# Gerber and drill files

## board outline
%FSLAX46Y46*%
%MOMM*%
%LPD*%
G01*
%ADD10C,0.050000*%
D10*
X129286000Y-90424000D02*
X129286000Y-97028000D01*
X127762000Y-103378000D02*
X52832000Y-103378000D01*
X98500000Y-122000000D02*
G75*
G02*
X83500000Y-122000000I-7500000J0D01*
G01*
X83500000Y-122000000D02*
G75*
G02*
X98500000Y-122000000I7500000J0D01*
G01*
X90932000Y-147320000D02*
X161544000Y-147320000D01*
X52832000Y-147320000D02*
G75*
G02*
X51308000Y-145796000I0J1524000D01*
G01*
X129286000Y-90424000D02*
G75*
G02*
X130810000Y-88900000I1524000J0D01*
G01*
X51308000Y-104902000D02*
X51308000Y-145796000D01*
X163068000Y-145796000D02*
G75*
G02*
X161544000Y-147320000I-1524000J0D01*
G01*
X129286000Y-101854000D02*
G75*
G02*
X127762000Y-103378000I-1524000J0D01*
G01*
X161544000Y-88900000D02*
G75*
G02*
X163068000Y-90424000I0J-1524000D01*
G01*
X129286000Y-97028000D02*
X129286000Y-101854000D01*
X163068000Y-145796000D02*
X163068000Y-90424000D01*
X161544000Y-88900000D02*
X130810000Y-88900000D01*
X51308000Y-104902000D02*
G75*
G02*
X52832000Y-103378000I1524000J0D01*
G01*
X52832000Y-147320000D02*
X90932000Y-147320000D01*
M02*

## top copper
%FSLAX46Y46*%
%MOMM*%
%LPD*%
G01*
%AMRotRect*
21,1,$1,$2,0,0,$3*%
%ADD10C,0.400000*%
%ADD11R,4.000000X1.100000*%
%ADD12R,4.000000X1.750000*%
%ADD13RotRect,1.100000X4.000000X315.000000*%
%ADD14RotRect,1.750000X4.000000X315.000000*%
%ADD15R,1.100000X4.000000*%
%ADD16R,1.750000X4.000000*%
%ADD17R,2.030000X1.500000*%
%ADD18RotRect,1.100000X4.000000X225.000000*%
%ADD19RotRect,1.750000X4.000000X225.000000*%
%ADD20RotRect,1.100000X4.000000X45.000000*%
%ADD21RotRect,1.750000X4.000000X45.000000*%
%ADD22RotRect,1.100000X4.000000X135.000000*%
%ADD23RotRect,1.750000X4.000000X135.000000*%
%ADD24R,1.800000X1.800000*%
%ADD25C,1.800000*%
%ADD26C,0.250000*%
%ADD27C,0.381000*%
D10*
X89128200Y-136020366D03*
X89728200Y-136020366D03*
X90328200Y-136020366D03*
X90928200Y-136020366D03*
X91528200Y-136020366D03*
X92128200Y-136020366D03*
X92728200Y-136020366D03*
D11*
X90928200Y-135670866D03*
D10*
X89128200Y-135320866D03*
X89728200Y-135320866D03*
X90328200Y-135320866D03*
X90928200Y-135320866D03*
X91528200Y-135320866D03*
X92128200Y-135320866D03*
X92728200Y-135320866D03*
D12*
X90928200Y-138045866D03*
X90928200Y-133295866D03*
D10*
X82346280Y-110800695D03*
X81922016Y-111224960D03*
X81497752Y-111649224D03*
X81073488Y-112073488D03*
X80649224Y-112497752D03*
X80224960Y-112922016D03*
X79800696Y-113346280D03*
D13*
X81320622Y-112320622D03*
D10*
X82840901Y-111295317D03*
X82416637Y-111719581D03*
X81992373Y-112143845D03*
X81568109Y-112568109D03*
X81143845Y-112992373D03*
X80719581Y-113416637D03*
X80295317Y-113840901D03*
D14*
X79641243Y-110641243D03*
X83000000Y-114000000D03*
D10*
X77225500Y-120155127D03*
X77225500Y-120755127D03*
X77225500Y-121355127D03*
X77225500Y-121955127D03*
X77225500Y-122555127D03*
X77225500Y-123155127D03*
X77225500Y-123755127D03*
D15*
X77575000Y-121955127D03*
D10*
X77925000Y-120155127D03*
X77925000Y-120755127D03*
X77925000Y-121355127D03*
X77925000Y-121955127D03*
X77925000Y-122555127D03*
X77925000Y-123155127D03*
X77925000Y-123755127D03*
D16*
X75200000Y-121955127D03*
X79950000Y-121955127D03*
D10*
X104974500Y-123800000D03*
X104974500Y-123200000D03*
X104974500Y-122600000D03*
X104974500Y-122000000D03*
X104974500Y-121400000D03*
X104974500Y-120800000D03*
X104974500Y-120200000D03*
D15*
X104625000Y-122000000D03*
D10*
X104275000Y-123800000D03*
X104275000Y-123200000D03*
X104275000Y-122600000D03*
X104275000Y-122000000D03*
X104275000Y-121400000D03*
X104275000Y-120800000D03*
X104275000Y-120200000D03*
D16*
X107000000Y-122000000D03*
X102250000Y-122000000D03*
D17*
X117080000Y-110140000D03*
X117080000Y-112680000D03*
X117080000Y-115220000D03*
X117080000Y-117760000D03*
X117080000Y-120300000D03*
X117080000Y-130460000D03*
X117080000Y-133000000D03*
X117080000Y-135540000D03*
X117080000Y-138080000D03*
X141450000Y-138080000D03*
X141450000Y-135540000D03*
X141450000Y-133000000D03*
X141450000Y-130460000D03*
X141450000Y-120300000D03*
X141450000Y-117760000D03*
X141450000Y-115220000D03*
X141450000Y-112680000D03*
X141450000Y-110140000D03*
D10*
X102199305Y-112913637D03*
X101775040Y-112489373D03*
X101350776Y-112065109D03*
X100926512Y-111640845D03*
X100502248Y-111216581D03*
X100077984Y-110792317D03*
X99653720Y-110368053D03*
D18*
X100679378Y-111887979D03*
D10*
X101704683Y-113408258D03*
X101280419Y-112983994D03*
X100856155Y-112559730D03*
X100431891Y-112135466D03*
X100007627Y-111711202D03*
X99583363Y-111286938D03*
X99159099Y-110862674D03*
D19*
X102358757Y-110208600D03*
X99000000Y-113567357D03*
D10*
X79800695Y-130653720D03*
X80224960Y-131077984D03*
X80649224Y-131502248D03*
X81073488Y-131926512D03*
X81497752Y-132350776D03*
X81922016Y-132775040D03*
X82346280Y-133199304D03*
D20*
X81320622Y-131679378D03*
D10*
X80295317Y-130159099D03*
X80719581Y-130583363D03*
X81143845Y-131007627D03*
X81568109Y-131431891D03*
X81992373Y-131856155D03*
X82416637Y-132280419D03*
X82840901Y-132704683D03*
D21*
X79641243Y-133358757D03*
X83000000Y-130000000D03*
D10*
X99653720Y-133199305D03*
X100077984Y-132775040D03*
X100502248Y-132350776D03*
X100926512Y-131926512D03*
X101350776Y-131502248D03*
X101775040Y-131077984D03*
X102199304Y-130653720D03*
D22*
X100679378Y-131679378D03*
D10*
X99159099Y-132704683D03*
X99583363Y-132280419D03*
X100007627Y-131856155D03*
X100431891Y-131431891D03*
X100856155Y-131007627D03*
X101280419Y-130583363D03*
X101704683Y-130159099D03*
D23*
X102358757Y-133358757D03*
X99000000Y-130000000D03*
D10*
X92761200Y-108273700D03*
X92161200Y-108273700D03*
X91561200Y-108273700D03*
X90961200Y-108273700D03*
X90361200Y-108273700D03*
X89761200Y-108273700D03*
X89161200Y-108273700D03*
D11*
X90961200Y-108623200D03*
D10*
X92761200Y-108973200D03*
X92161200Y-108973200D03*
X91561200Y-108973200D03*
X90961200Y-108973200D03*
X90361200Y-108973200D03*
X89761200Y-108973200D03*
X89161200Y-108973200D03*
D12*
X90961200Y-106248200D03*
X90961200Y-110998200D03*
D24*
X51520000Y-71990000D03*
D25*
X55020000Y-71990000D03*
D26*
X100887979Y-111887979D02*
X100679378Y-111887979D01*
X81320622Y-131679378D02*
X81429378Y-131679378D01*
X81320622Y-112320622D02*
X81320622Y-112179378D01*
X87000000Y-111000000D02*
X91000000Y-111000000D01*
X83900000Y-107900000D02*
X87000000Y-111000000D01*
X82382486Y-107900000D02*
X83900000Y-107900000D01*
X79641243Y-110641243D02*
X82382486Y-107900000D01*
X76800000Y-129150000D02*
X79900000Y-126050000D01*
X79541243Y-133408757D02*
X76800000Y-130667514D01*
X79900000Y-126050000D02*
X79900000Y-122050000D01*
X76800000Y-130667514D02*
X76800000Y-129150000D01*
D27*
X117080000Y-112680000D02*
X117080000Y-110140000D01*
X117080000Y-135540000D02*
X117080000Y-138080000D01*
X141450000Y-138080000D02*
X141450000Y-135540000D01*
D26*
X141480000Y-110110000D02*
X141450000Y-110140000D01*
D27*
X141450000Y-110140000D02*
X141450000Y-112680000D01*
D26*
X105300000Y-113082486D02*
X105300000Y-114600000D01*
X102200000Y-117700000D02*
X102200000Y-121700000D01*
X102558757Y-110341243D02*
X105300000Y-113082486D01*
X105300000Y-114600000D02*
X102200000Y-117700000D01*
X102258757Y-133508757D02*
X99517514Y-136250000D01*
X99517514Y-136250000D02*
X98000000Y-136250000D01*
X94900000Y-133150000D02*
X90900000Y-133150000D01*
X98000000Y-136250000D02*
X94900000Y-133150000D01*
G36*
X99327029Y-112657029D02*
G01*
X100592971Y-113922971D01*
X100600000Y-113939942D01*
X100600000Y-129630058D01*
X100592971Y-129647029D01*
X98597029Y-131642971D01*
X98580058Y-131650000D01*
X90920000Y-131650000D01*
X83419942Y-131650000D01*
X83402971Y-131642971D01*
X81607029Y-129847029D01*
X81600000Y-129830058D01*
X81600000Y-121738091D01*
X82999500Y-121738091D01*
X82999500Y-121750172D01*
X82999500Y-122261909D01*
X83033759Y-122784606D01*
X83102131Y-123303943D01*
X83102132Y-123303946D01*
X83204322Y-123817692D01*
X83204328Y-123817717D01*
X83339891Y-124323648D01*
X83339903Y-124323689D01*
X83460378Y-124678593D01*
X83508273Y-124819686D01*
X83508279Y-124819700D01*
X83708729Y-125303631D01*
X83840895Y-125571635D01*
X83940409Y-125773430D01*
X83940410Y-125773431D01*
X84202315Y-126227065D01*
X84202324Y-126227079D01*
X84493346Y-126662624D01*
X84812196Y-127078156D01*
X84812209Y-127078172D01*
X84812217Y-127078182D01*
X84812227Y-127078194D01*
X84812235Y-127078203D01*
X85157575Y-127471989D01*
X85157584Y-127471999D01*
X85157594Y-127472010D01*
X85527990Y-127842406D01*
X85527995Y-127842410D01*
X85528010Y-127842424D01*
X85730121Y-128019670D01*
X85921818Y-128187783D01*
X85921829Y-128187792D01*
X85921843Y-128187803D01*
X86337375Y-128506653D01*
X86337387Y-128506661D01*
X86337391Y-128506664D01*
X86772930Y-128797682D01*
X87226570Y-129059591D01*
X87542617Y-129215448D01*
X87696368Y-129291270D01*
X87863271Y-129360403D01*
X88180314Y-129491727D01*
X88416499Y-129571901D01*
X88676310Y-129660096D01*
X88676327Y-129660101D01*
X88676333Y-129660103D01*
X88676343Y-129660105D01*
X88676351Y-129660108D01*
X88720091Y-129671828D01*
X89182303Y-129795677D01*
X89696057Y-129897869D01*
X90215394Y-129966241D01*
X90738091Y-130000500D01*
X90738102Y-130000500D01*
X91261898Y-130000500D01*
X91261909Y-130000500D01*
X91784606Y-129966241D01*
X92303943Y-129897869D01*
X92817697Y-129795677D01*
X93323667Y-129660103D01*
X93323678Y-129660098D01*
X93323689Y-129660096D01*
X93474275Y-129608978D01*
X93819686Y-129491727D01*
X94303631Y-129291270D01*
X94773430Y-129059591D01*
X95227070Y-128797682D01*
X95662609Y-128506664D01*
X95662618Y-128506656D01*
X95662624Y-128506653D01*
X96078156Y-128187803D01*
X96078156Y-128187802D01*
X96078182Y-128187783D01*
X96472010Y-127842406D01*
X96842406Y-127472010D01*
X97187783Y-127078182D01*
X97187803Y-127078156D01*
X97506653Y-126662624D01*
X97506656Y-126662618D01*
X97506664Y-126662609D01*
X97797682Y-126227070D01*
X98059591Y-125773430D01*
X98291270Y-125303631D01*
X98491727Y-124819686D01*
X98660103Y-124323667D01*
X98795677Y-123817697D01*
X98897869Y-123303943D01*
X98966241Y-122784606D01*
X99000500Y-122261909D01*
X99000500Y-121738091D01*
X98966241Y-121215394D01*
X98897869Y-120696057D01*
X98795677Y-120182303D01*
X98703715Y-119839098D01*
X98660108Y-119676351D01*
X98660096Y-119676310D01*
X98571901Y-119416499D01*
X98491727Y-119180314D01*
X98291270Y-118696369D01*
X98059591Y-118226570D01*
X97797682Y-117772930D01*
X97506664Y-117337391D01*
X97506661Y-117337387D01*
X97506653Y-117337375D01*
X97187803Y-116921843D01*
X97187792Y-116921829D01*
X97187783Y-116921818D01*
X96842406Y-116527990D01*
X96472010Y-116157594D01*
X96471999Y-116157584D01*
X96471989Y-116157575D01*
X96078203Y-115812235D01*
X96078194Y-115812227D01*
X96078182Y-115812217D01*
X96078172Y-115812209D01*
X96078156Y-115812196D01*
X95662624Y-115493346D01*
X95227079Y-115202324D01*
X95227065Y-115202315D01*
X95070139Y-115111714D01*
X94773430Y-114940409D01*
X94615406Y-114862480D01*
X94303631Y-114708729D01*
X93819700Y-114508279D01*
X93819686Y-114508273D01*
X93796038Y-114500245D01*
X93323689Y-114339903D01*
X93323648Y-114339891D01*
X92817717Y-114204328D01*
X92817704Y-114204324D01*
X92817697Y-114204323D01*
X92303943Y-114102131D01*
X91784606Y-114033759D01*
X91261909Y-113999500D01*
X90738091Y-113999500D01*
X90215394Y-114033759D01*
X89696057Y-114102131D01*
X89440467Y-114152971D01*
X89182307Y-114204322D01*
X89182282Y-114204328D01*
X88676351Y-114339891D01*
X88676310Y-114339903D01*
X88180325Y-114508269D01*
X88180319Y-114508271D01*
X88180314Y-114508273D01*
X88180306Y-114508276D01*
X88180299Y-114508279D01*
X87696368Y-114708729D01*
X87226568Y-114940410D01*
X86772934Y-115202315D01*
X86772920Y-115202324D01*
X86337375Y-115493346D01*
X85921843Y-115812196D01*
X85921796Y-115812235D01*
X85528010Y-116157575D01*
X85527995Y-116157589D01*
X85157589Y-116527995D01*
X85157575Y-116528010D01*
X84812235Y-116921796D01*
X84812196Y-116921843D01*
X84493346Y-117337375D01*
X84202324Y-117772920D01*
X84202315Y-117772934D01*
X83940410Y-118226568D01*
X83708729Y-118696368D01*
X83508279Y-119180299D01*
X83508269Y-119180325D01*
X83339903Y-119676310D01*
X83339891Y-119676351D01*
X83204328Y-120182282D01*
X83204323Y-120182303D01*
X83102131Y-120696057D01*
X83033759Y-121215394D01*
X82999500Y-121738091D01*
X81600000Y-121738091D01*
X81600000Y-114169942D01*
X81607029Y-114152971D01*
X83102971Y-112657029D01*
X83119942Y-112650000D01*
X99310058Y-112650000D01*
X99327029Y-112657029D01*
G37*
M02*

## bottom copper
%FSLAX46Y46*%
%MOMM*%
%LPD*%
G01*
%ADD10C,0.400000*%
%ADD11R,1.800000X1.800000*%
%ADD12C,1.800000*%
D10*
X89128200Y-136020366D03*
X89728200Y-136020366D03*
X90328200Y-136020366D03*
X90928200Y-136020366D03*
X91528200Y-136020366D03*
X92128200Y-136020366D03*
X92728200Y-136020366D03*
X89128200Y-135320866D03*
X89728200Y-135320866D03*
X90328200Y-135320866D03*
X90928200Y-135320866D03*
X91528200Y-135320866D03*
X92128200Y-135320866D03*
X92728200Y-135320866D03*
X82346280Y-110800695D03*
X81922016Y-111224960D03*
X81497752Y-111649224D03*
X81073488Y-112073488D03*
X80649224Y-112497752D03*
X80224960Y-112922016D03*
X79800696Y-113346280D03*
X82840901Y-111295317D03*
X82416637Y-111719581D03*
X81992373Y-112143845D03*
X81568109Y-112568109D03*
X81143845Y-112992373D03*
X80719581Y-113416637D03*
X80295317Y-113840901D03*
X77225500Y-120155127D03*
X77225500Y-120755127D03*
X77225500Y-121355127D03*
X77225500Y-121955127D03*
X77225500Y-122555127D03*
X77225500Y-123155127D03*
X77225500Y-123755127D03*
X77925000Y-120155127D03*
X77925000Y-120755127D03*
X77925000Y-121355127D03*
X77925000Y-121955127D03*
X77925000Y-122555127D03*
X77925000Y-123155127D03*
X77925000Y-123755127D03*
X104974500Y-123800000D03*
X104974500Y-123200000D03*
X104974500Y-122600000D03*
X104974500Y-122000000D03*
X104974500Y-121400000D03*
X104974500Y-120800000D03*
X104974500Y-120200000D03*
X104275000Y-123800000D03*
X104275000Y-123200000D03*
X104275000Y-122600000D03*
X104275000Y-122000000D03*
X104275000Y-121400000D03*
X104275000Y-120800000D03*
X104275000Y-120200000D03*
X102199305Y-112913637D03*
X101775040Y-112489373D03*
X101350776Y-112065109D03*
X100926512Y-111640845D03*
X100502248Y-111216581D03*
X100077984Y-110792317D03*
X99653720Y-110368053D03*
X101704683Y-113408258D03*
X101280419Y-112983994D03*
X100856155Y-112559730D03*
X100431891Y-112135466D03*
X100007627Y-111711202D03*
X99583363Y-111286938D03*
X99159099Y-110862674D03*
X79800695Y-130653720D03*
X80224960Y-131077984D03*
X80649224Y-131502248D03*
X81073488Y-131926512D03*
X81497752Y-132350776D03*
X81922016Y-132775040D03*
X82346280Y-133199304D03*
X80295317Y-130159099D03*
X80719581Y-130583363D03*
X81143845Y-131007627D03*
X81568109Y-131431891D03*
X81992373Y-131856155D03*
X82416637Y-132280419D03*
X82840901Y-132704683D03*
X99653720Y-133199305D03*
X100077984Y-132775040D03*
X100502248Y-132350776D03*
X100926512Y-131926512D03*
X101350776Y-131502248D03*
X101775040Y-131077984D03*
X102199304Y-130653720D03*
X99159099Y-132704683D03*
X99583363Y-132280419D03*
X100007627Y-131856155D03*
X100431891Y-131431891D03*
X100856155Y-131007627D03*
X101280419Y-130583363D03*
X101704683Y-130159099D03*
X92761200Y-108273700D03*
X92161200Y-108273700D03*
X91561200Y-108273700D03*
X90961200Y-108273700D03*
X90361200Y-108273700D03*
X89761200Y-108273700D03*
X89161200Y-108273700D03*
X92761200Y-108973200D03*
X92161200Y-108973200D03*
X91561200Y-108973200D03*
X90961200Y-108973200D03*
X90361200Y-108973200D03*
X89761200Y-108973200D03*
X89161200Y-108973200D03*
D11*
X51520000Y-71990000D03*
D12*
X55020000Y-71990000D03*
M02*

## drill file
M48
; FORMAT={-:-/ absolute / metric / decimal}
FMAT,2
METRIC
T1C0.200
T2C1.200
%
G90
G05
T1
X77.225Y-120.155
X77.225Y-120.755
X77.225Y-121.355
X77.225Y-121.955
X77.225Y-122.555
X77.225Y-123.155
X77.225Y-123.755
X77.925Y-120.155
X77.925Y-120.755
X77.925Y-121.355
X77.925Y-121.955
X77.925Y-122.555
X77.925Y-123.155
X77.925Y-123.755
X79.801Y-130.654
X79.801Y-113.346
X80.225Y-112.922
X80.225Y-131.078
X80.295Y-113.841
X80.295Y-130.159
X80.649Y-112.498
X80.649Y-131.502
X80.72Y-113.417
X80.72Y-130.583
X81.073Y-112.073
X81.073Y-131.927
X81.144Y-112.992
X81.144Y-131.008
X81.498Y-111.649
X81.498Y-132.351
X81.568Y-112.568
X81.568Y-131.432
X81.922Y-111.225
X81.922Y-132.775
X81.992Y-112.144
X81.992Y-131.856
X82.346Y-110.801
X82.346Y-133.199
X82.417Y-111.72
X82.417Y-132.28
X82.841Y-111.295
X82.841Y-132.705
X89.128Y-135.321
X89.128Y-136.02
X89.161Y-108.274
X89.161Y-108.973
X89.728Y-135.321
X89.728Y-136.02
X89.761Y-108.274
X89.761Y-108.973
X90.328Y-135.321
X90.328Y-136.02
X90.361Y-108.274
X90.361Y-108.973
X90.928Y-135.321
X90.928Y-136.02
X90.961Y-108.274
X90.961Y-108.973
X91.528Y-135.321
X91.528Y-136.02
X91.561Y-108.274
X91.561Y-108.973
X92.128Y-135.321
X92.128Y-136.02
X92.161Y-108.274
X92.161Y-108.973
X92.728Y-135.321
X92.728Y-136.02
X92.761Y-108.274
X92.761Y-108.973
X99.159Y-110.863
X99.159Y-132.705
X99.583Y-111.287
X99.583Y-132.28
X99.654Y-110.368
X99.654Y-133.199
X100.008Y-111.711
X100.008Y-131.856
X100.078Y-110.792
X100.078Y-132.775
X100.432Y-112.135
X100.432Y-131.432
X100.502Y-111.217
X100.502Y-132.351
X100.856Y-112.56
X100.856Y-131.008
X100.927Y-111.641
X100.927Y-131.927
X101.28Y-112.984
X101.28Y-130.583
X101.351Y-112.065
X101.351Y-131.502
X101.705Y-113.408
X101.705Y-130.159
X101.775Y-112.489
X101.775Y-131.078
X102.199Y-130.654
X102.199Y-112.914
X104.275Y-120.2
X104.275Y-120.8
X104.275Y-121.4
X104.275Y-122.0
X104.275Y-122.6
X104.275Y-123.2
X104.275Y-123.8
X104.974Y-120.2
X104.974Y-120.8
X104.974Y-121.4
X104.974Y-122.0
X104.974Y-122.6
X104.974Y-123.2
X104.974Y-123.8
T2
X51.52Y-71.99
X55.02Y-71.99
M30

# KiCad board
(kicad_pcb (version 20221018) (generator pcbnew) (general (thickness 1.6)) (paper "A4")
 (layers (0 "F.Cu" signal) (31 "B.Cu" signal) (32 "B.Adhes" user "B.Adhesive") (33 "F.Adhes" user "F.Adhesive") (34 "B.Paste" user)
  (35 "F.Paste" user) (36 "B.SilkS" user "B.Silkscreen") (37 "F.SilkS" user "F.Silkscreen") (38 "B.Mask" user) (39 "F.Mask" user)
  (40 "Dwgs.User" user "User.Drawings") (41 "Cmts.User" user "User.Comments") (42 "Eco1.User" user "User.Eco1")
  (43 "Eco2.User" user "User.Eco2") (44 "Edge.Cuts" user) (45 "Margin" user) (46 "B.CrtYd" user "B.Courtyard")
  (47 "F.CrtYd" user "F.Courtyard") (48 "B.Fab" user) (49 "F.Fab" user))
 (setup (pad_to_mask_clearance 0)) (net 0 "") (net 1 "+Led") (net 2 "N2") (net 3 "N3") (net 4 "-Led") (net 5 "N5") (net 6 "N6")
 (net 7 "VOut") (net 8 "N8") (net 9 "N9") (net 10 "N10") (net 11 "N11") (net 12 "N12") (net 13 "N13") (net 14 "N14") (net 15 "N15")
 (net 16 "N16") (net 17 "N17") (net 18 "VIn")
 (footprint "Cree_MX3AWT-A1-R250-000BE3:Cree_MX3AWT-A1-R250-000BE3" (layer "F.Cu") (at 85.9282 138.045866 90)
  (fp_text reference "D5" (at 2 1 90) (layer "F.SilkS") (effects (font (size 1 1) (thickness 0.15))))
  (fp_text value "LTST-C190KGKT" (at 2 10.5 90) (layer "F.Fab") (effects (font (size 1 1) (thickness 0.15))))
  (pad "65" thru_hole circle (at 2.0255 3.2 90) (size 0.4 0.4) (drill 0.2) (layers "*.Cu" "B.Mask"))
  (pad "65" thru_hole circle (at 2.0255 3.8 90) (size 0.4 0.4) (drill 0.2) (layers "*.Cu" "B.Mask"))
  (pad "65" thru_hole circle (at 2.0255 4.4 90) (size 0.4 0.4) (drill 0.2) (layers "*.Cu" "B.Mask"))
  (pad "65" thru_hole circle (at 2.0255 5 90) (size 0.4 0.4) (drill 0.2) (layers "*.Cu" "B.Mask"))
  (pad "65" thru_hole circle (at 2.0255 5.6 90) (size 0.4 0.4) (drill 0.2) (layers "*.Cu" "B.Mask"))
  (pad "65" thru_hole circle (at 2.0255 6.2 90) (size 0.4 0.4) (drill 0.2) (layers "*.Cu" "B.Mask"))
  (pad "65" thru_hole circle (at 2.0255 6.8 90) (size 0.4 0.4) (drill 0.2) (layers "*.Cu" "B.Mask"))
  (pad "65" smd rect (at 2.375 5 90) (size 1.1 4) (layers "F.Cu" "F.Paste" "F.Mask"))
  (pad "65" thru_hole circle (at 2.725 3.2 90) (size 0.4 0.4) (drill 0.2) (layers "*.Cu" "B.Mask"))
  (pad "65" thru_hole circle (at 2.725 3.8 90) (size 0.4 0.4) (drill 0.2) (layers "*.Cu" "B.Mask"))
  (pad "65" thru_hole circle (at 2.725 4.4 90) (size 0.4 0.4) (drill 0.2) (layers "*.Cu" "B.Mask"))
  (pad "65" thru_hole circle (at 2.725 5 90) (size 0.4 0.4) (drill 0.2) (layers "*.Cu" "B.Mask"))
  (pad "65" thru_hole circle (at 2.725 5.6 90) (size 0.4 0.4) (drill 0.2) (layers "*.Cu" "B.Mask"))
  (pad "65" thru_hole circle (at 2.725 6.2 90) (size 0.4 0.4) (drill 0.2) (layers "*.Cu" "B.Mask"))
  (pad "65" thru_hole circle (at 2.725 6.8 90) (size 0.4 0.4) (drill 0.2) (layers "*.Cu" "B.Mask"))
  (pad "A" smd rect (at 0 5 90) (size 1.75 4) (layers "F.Cu" "F.Paste" "F.Mask") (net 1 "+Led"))
  (pad "C" smd rect (at 4.75 5 90) (size 1.75 4) (layers "F.Cu" "F.Paste" "F.Mask") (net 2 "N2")))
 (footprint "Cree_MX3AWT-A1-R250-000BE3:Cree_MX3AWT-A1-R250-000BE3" (layer "F.Cu") (at 83.176777 107.105709 -45)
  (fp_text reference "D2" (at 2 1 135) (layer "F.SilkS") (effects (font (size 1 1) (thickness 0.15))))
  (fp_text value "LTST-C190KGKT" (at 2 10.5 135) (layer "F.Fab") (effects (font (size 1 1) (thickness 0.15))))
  (pad "65" thru_hole circle (at 2.0255 3.2 315) (size 0.4 0.4) (drill 0.2) (layers "*.Cu" "B.Mask"))
  (pad "65" thru_hole circle (at 2.0255 3.8 315) (size 0.4 0.4) (drill 0.2) (layers "*.Cu" "B.Mask"))
  (pad "65" thru_hole circle (at 2.0255 4.4 315) (size 0.4 0.4) (drill 0.2) (layers "*.Cu" "B.Mask"))
  (pad "65" thru_hole circle (at 2.0255 5 315) (size 0.4 0.4) (drill 0.2) (layers "*.Cu" "B.Mask"))
  (pad "65" thru_hole circle (at 2.0255 5.6 315) (size 0.4 0.4) (drill 0.2) (layers "*.Cu" "B.Mask"))
  (pad "65" thru_hole circle (at 2.0255 6.2 315) (size 0.4 0.4) (drill 0.2) (layers "*.Cu" "B.Mask"))
  (pad "65" thru_hole circle (at 2.0255 6.8 315) (size 0.4 0.4) (drill 0.2) (layers "*.Cu" "B.Mask"))
  (pad "65" smd rect (at 2.375001 5 315) (size 1.1 4) (layers "F.Cu" "F.Paste" "F.Mask"))
  (pad "65" thru_hole circle (at 2.725 3.2 315) (size 0.4 0.4) (drill 0.2) (layers "*.Cu" "B.Mask"))
  (pad "65" thru_hole circle (at 2.725 3.8 315) (size 0.4 0.4) (drill 0.2) (layers "*.Cu" "B.Mask"))
  (pad "65" thru_hole circle (at 2.725 4.4 315) (size 0.4 0.4) (drill 0.2) (layers "*.Cu" "B.Mask"))
  (pad "65" thru_hole circle (at 2.725 5 315) (size 0.4 0.4) (drill 0.2) (layers "*.Cu" "B.Mask"))
  (pad "65" thru_hole circle (at 2.725 5.6 315) (size 0.4 0.4) (drill 0.2) (layers "*.Cu" "B.Mask"))
  (pad "65" thru_hole circle (at 2.725 6.2 315) (size 0.4 0.4) (drill 0.2) (layers "*.Cu" "B.Mask"))
  (pad "65" thru_hole circle (at 2.725 6.8 315) (size 0.4 0.4) (drill 0.2) (layers "*.Cu" "B.Mask"))
  (pad "A" smd rect (at 0 5 315) (size 1.75 4) (layers "F.Cu" "F.Paste" "F.Mask") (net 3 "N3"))
  (pad "C" smd rect (at 4.75 5 315) (size 1.75 4) (layers "F.Cu" "F.Paste" "F.Mask") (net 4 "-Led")))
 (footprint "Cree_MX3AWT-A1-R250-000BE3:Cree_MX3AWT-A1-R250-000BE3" (layer "F.Cu") (at 75.2 116.955127)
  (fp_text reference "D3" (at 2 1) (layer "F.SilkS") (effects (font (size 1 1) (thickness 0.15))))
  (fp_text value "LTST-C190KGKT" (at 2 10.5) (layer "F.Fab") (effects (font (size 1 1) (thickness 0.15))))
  (pad "65" thru_hole circle (at 2.0255 3.2) (size 0.4 0.4) (drill 0.2) (layers "*.Cu" "B.Mask"))
  (pad "65" thru_hole circle (at 2.0255 3.8) (size 0.4 0.4) (drill 0.2) (layers "*.Cu" "B.Mask"))
  (pad "65" thru_hole circle (at 2.0255 4.4) (size 0.4 0.4) (drill 0.2) (layers "*.Cu" "B.Mask"))
  (pad "65" thru_hole circle (at 2.0255 5) (size 0.4 0.4) (drill 0.2) (layers "*.Cu" "B.Mask"))
  (pad "65" thru_hole circle (at 2.0255 5.6) (size 0.4 0.4) (drill 0.2) (layers "*.Cu" "B.Mask"))
  (pad "65" thru_hole circle (at 2.0255 6.2) (size 0.4 0.4) (drill 0.2) (layers "*.Cu" "B.Mask"))
  (pad "65" thru_hole circle (at 2.0255 6.8) (size 0.4 0.4) (drill 0.2) (layers "*.Cu" "B.Mask"))
  (pad "65" smd rect (at 2.375 5) (size 1.1 4) (layers "F.Cu" "F.Paste" "F.Mask"))
  (pad "65" thru_hole circle (at 2.725 3.2) (size 0.4 0.4) (drill 0.2) (layers "*.Cu" "B.Mask"))
  (pad "65" thru_hole circle (at 2.725 3.8) (size 0.4 0.4) (drill 0.2) (layers "*.Cu" "B.Mask"))
  (pad "65" thru_hole circle (at 2.725 4.4) (size 0.4 0.4) (drill 0.2) (layers "*.Cu" "B.Mask"))
  (pad "65" thru_hole circle (at 2.725 5) (size 0.4 0.4) (drill 0.2) (layers "*.Cu" "B.Mask"))
  (pad "65" thru_hole circle (at 2.725 5.6) (size 0.4 0.4) (drill 0.2) (layers "*.Cu" "B.Mask"))
  (pad "65" thru_hole circle (at 2.725 6.2) (size 0.4 0.4) (drill 0.2) (layers "*.Cu" "B.Mask"))
  (pad "65" thru_hole circle (at 2.725 6.8) (size 0.4 0.4) (drill 0.2) (layers "*.Cu" "B.Mask"))
  (pad "A" smd rect (at 0 5) (size 1.75 4) (layers "F.Cu" "F.Paste" "F.Mask") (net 1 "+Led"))
  (pad "C" smd rect (at 4.75 5) (size 1.75 4) (layers "F.Cu" "F.Paste" "F.Mask") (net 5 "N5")))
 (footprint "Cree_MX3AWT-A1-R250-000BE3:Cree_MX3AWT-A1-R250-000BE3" (layer "F.Cu") (at 107 127 180)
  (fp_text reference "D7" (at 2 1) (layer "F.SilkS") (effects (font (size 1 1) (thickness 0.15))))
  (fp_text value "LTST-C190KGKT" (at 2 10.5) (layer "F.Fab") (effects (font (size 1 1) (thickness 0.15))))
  (pad "65" thru_hole circle (at 2.0255 3.2 180) (size 0.4 0.4) (drill 0.2) (layers "*.Cu" "B.Mask"))
  (pad "65" thru_hole circle (at 2.0255 3.8 180) (size 0.4 0.4) (drill 0.2) (layers "*.Cu" "B.Mask"))
  (pad "65" thru_hole circle (at 2.0255 4.4 180) (size 0.4 0.4) (drill 0.2) (layers "*.Cu" "B.Mask"))
  (pad "65" thru_hole circle (at 2.0255 5 180) (size 0.4 0.4) (drill 0.2) (layers "*.Cu" "B.Mask"))
  (pad "65" thru_hole circle (at 2.0255 5.6 180) (size 0.4 0.4) (drill 0.2) (layers "*.Cu" "B.Mask"))
  (pad "65" thru_hole circle (at 2.0255 6.2 180) (size 0.4 0.4) (drill 0.2) (layers "*.Cu" "B.Mask"))
  (pad "65" thru_hole circle (at 2.0255 6.8 180) (size 0.4 0.4) (drill 0.2) (layers "*.Cu" "B.Mask"))
  (pad "65" smd rect (at 2.375 5 180) (size 1.1 4) (layers "F.Cu" "F.Paste" "F.Mask"))
  (pad "65" thru_hole circle (at 2.725 3.2 180) (size 0.4 0.4) (drill 0.2) (layers "*.Cu" "B.Mask"))
  (pad "65" thru_hole circle (at 2.725 3.8 180) (size 0.4 0.4) (drill 0.2) (layers "*.Cu" "B.Mask"))
  (pad "65" thru_hole circle (at 2.725 4.4 180) (size 0.4 0.4) (drill 0.2) (layers "*.Cu" "B.Mask"))
  (pad "65" thru_hole circle (at 2.725 5 180) (size 0.4 0.4) (drill 0.2) (layers "*.Cu" "B.Mask"))
  (pad "65" thru_hole circle (at 2.725 5.6 180) (size 0.4 0.4) (drill 0.2) (layers "*.Cu" "B.Mask"))
  (pad "65" thru_hole circle (at 2.725 6.2 180) (size 0.4 0.4) (drill 0.2) (layers "*.Cu" "B.Mask"))
  (pad "65" thru_hole circle (at 2.725 6.8 180) (size 0.4 0.4) (drill 0.2) (layers "*.Cu" "B.Mask"))
  (pad "A" smd rect (at 0 5 180) (size 1.75 4) (layers "F.Cu" "F.Paste" "F.Mask") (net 1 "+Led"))
  (pad "C" smd rect (at 4.75 5 180) (size 1.75 4) (layers "F.Cu" "F.Paste" "F.Mask") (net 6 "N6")))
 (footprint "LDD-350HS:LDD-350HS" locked (layer "F.Cu") (at 117.08 105.64)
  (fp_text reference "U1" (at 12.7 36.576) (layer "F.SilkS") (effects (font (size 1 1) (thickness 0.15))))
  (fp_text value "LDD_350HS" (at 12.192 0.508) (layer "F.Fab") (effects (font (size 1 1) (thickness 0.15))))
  (pad "1" smd rect locked (at 0 4.5) (size 2.03 1.5) (layers "F.Cu" "F.Paste" "F.Mask") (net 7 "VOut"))
  (pad "2" smd rect locked (at 0 7.04) (size 2.03 1.5) (layers "F.Cu" "F.Paste" "F.Mask") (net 7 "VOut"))
  (pad "3" smd rect locked (at 0 9.58) (size 2.03 1.5) (layers "F.Cu" "F.Paste" "F.Mask") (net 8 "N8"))
  (pad "4" smd rect locked (at 0 12.12) (size 2.03 1.5) (layers "F.Cu" "F.Paste" "F.Mask") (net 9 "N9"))
  (pad "5" smd rect locked (at 0 14.66) (size 2.03 1.5) (layers "F.Cu" "F.Paste" "F.Mask") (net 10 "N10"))
  (pad "9" smd rect locked (at 0 24.82) (size 2.03 1.5) (layers "F.Cu" "F.Paste" "F.Mask") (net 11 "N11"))
  (pad "10" smd rect locked (at 0 27.36) (size 2.03 1.5) (layers "F.Cu" "F.Paste" "F.Mask") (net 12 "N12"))
  (pad "11" smd rect locked (at 0 29.9) (size 2.03 1.5) (layers "F.Cu" "F.Paste" "F.Mask") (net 4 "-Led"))
  (pad "12" smd rect locked (at 0 32.44) (size 2.03 1.5) (layers "F.Cu" "F.Paste" "F.Mask") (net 4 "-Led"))
  (pad "13" smd rect locked (at 24.37 32.44) (size 2.03 1.5) (layers "F.Cu" "F.Paste" "F.Mask") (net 1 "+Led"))
  (pad "14" smd rect locked (at 24.37 29.9) (size 2.03 1.5) (layers "F.Cu" "F.Paste" "F.Mask") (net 1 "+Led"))
  (pad "15" smd rect locked (at 24.37 27.36) (size 2.03 1.5) (layers "F.Cu" "F.Paste" "F.Mask") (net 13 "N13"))
  (pad "16" smd rect locked (at 24.37 24.82) (size 2.03 1.5) (layers "F.Cu" "F.Paste" "F.Mask") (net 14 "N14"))
  (pad "20" smd rect locked (at 24.37 14.66) (size 2.03 1.5) (layers "F.Cu" "F.Paste" "F.Mask") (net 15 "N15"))
  (pad "21" smd rect locked (at 24.37 12.12) (size 2.03 1.5) (layers "F.Cu" "F.Paste" "F.Mask") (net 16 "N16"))
  (pad "22" smd rect locked (at 24.37 9.58) (size 2.03 1.5) (layers "F.Cu" "F.Paste" "F.Mask") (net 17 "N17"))
  (pad "23" smd rect locked (at 24.37 7.04) (size 2.03 1.5) (layers "F.Cu" "F.Paste" "F.Mask") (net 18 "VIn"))
  (pad "24" smd rect locked (at 24.37 4.5) (size 2.03 1.5) (layers "F.Cu" "F.Paste" "F.Mask") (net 18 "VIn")))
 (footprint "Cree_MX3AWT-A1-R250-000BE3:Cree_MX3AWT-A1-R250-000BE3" (layer "F.Cu") (at 105.894291 113.744134 -135)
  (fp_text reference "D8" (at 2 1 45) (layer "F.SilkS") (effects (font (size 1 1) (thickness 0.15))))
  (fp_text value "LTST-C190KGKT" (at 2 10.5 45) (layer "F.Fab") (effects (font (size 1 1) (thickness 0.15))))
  (pad "65" thru_hole circle (at 2.0255 3.2 225) (size 0.4 0.4) (drill 0.2) (layers "*.Cu" "B.Mask"))
  (pad "65" thru_hole circle (at 2.0255 3.8 225) (size 0.4 0.4) (drill 0.2) (layers "*.Cu" "B.Mask"))
  (pad "65" thru_hole circle (at 2.0255 4.4 225) (size 0.4 0.4) (drill 0.2) (layers "*.Cu" "B.Mask"))
  (pad "65" thru_hole circle (at 2.0255 5 225) (size 0.4 0.4) (drill 0.2) (layers "*.Cu" "B.Mask"))
  (pad "65" thru_hole circle (at 2.0255 5.6 225) (size 0.4 0.4) (drill 0.2) (layers "*.Cu" "B.Mask"))
  (pad "65" thru_hole circle (at 2.0255 6.2 225) (size 0.4 0.4) (drill 0.2) (layers "*.Cu" "B.Mask"))
  (pad "65" thru_hole circle (at 2.0255 6.8 225) (size 0.4 0.4) (drill 0.2) (layers "*.Cu" "B.Mask"))
  (pad "65" smd rect (at 2.375001 5 225) (size 1.1 4) (layers "F.Cu" "F.Paste" "F.Mask"))
  (pad "65" thru_hole circle (at 2.725 3.2 225) (size 0.4 0.4) (drill 0.2) (layers "*.Cu" "B.Mask"))
  (pad "65" thru_hole circle (at 2.725 3.8 225) (size 0.4 0.4) (drill 0.2) (layers "*.Cu" "B.Mask"))
  (pad "65" thru_hole circle (at 2.725 4.4 225) (size 0.4 0.4) (drill 0.2) (layers "*.Cu" "B.Mask"))
  (pad "65" thru_hole circle (at 2.725 5 225) (size 0.4 0.4) (drill 0.2) (layers "*.Cu" "B.Mask"))
  (pad "65" thru_hole circle (at 2.725 5.6 225) (size 0.4 0.4) (drill 0.2) (layers "*.Cu" "B.Mask"))
  (pad "65" thru_hole circle (at 2.725 6.2 225) (size 0.4 0.4) (drill 0.2) (layers "*.Cu" "B.Mask"))
  (pad "65" thru_hole circle (at 2.725 6.8 225) (size 0.4 0.4) (drill 0.2) (layers "*.Cu" "B.Mask"))
  (pad "A" smd rect (at 0 5 225) (size 1.75 4) (layers "F.Cu" "F.Paste" "F.Mask") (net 6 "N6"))
  (pad "C" smd rect (at 4.75 5 225) (size 1.75 4) (layers "F.Cu" "F.Paste" "F.Mask") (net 4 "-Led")))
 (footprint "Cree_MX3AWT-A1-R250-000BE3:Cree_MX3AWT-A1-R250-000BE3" (layer "F.Cu") (at 76.105709 129.823223 45)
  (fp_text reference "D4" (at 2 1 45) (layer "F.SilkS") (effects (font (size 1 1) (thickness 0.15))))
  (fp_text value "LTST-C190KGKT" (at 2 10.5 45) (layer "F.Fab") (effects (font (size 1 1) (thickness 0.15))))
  (pad "65" thru_hole circle (at 2.0255 3.2 45) (size 0.4 0.4) (drill 0.2) (layers "*.Cu" "B.Mask"))
  (pad "65" thru_hole circle (at 2.0255 3.8 45) (size 0.4 0.4) (drill 0.2) (layers "*.Cu" "B.Mask"))
  (pad "65" thru_hole circle (at 2.0255 4.4 45) (size 0.4 0.4) (drill 0.2) (layers "*.Cu" "B.Mask"))
  (pad "65" thru_hole circle (at 2.0255 5 45) (size 0.4 0.4) (drill 0.2) (layers "*.Cu" "B.Mask"))
  (pad "65" thru_hole circle (at 2.0255 5.6 45) (size 0.4 0.4) (drill 0.2) (layers "*.Cu" "B.Mask"))
  (pad "65" thru_hole circle (at 2.0255 6.2 45) (size 0.4 0.4) (drill 0.2) (layers "*.Cu" "B.Mask"))
  (pad "65" thru_hole circle (at 2.0255 6.8 45) (size 0.4 0.4) (drill 0.2) (layers "*.Cu" "B.Mask"))
  (pad "65" smd rect (at 2.375001 5 45) (size 1.1 4) (layers "F.Cu" "F.Paste" "F.Mask"))
  (pad "65" thru_hole circle (at 2.725 3.2 45) (size 0.4 0.4) (drill 0.2) (layers "*.Cu" "B.Mask"))
  (pad "65" thru_hole circle (at 2.725 3.8 45) (size 0.4 0.4) (drill 0.2) (layers "*.Cu" "B.Mask"))
  (pad "65" thru_hole circle (at 2.725 4.4 45) (size 0.4 0.4) (drill 0.2) (layers "*.Cu" "B.Mask"))
  (pad "65" thru_hole circle (at 2.725 5 45) (size 0.4 0.4) (drill 0.2) (layers "*.Cu" "B.Mask"))
  (pad "65" thru_hole circle (at 2.725 5.6 45) (size 0.4 0.4) (drill 0.2) (layers "*.Cu" "B.Mask"))
  (pad "65" thru_hole circle (at 2.725 6.2 45) (size 0.4 0.4) (drill 0.2) (layers "*.Cu" "B.Mask"))
  (pad "65" thru_hole circle (at 2.725 6.8 45) (size 0.4 0.4) (drill 0.2) (layers "*.Cu" "B.Mask"))
  (pad "A" smd rect (at 0 5 45) (size 1.75 4) (layers "F.Cu" "F.Paste" "F.Mask") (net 5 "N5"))
  (pad "C" smd rect (at 4.75 5 45) (size 1.75 4) (layers "F.Cu" "F.Paste" "F.Mask") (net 4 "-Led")))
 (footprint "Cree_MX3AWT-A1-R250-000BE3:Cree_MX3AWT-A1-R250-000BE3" (layer "F.Cu") (at 98.823223 136.894291 135)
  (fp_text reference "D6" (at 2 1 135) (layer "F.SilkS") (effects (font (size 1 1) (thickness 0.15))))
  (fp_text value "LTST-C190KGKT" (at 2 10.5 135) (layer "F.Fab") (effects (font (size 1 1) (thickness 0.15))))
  (pad "65" thru_hole circle (at 2.0255 3.2 135) (size 0.4 0.4) (drill 0.2) (layers "*.Cu" "B.Mask"))
  (pad "65" thru_hole circle (at 2.0255 3.8 135) (size 0.4 0.4) (drill 0.2) (layers "*.Cu" "B.Mask"))
  (pad "65" thru_hole circle (at 2.0255 4.4 135) (size 0.4 0.4) (drill 0.2) (layers "*.Cu" "B.Mask"))
  (pad "65" thru_hole circle (at 2.0255 5 135) (size 0.4 0.4) (drill 0.2) (layers "*.Cu" "B.Mask"))
  (pad "65" thru_hole circle (at 2.0255 5.6 135) (size 0.4 0.4) (drill 0.2) (layers "*.Cu" "B.Mask"))
  (pad "65" thru_hole circle (at 2.0255 6.2 135) (size 0.4 0.4) (drill 0.2) (layers "*.Cu" "B.Mask"))
  (pad "65" thru_hole circle (at 2.0255 6.8 135) (size 0.4 0.4) (drill 0.2) (layers "*.Cu" "B.Mask"))
  (pad "65" smd rect (at 2.375001 5 135) (size 1.1 4) (layers "F.Cu" "F.Paste" "F.Mask"))
  (pad "65" thru_hole circle (at 2.725 3.2 135) (size 0.4 0.4) (drill 0.2) (layers "*.Cu" "B.Mask"))
  (pad "65" thru_hole circle (at 2.725 3.8 135) (size 0.4 0.4) (drill 0.2) (layers "*.Cu" "B.Mask"))
  (pad "65" thru_hole circle (at 2.725 4.4 135) (size 0.4 0.4) (drill 0.2) (layers "*.Cu" "B.Mask"))
  (pad "65" thru_hole circle (at 2.725 5 135) (size 0.4 0.4) (drill 0.2) (layers "*.Cu" "B.Mask"))
  (pad "65" thru_hole circle (at 2.725 5.6 135) (size 0.4 0.4) (drill 0.2) (layers "*.Cu" "B.Mask"))
  (pad "65" thru_hole circle (at 2.725 6.2 135) (size 0.4 0.4) (drill 0.2) (layers "*.Cu" "B.Mask"))
  (pad "65" thru_hole circle (at 2.725 6.8 135) (size 0.4 0.4) (drill 0.2) (layers "*.Cu" "B.Mask"))
  (pad "A" smd rect (at 0 5 135) (size 1.75 4) (layers "F.Cu" "F.Paste" "F.Mask") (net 2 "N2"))
  (pad "C" smd rect (at 4.75 5 135) (size 1.75 4) (layers "F.Cu" "F.Paste" "F.Mask") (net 4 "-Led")))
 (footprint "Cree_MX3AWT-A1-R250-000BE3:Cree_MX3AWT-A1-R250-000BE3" (layer "F.Cu") (at 95.9612 106.2482 -90)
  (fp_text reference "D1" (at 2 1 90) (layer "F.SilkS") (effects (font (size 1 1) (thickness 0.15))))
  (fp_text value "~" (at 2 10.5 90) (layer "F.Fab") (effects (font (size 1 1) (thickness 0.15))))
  (pad "65" thru_hole circle (at 2.0255 3.2 270) (size 0.4 0.4) (drill 0.2) (layers "*.Cu" "B.Mask"))
  (pad "65" thru_hole circle (at 2.0255 3.8 270) (size 0.4 0.4) (drill 0.2) (layers "*.Cu" "B.Mask"))
  (pad "65" thru_hole circle (at 2.0255 4.4 270) (size 0.4 0.4) (drill 0.2) (layers "*.Cu" "B.Mask"))
  (pad "65" thru_hole circle (at 2.0255 5 270) (size 0.4 0.4) (drill 0.2) (layers "*.Cu" "B.Mask"))
  (pad "65" thru_hole circle (at 2.0255 5.6 270) (size 0.4 0.4) (drill 0.2) (layers "*.Cu" "B.Mask"))
  (pad "65" thru_hole circle (at 2.0255 6.2 270) (size 0.4 0.4) (drill 0.2) (layers "*.Cu" "B.Mask"))
  (pad "65" thru_hole circle (at 2.0255 6.8 270) (size 0.4 0.4) (drill 0.2) (layers "*.Cu" "B.Mask"))
  (pad "65" smd rect (at 2.375 5 270) (size 1.1 4) (layers "F.Cu" "F.Paste" "F.Mask"))
  (pad "65" thru_hole circle (at 2.725 3.2 270) (size 0.4 0.4) (drill 0.2) (layers "*.Cu" "B.Mask"))
  (pad "65" thru_hole circle (at 2.725 3.8 270) (size 0.4 0.4) (drill 0.2) (layers "*.Cu" "B.Mask"))
  (pad "65" thru_hole circle (at 2.725 4.4 270) (size 0.4 0.4) (drill 0.2) (layers "*.Cu" "B.Mask"))
  (pad "65" thru_hole circle (at 2.725 5 270) (size 0.4 0.4) (drill 0.2) (layers "*.Cu" "B.Mask"))
  (pad "65" thru_hole circle (at 2.725 5.6 270) (size 0.4 0.4) (drill 0.2) (layers "*.Cu" "B.Mask"))
  (pad "65" thru_hole circle (at 2.725 6.2 270) (size 0.4 0.4) (drill 0.2) (layers "*.Cu" "B.Mask"))
  (pad "65" thru_hole circle (at 2.725 6.8 270) (size 0.4 0.4) (drill 0.2) (layers "*.Cu" "B.Mask"))
  (pad "A" smd rect (at 0 5 270) (size 1.75 4) (layers "F.Cu" "F.Paste" "F.Mask") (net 1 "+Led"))
  (pad "C" smd rect (at 4.75 5 270) (size 1.75 4) (layers "F.Cu" "F.Paste" "F.Mask") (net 3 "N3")))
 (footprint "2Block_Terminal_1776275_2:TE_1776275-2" (layer "F.Cu") (at 51.52 71.99)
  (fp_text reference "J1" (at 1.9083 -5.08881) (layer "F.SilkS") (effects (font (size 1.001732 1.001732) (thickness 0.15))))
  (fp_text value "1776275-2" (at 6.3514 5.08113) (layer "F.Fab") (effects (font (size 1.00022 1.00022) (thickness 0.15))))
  (pad "1" thru_hole rect (at 0 0) (size 1.8 1.8) (drill 1.2) (layers "*.Cu" "*.Mask") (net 18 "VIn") (solder_mask_margin 0.102))
  (pad "2" thru_hole circle (at 3.5 0) (size 1.8 1.8) (drill 1.2) (layers "*.Cu" "*.Mask") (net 7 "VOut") (solder_mask_margin 0.102)))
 (gr_line (start 129.286 90.424) (end 129.286 97.028) (stroke (width 0.05) (type solid)) (layer "Edge.Cuts"))
 (gr_line (start 127.762 103.378) (end 52.832 103.378) (stroke (width 0.05) (type solid)) (layer "Edge.Cuts"))
 (gr_circle (center 91 122) (end 98.5 122) (stroke (width 0.05) (type solid)) (fill none) (layer "Edge.Cuts"))
 (gr_line (start 90.932 147.32) (end 161.544 147.32) (stroke (width 0.05) (type solid)) (layer "Edge.Cuts"))
 (gr_arc (start 52.832 147.32) (mid 51.754369 146.873631) (end 51.308 145.796) (stroke (width 0.05) (type solid)) (layer "Edge.Cuts"))
 (gr_arc (start 129.286 90.424) (mid 129.732369 89.346369) (end 130.81 88.9) (stroke (width 0.05) (type solid)) (layer "Edge.Cuts"))
 (gr_line (start 51.308 104.902) (end 51.308 145.796) (stroke (width 0.05) (type solid)) (layer "Edge.Cuts"))
 (gr_arc (start 163.068 145.796) (mid 162.621631 146.873631) (end 161.544 147.32) (stroke (width 0.05) (type solid)) (layer "Edge.Cuts"))
 (gr_arc (start 129.286 101.854) (mid 128.839631 102.931631) (end 127.762 103.378) (stroke (width 0.05) (type solid)) (layer "Edge.Cuts"))
 (gr_arc (start 161.544 88.9) (mid 162.621631 89.346369) (end 163.068 90.424) (stroke (width 0.05) (type solid)) (layer "Edge.Cuts"))
 (gr_line (start 129.286 97.028) (end 129.286 101.854) (stroke (width 0.05) (type solid)) (layer "Edge.Cuts"))
 (gr_line (start 163.068 145.796) (end 163.068 90.424) (stroke (width 0.05) (type solid)) (layer "Edge.Cuts"))
 (gr_line (start 161.544 88.9) (end 130.81 88.9) (stroke (width 0.05) (type solid)) (layer "Edge.Cuts"))
 (gr_arc (start 51.308 104.902) (mid 51.754369 103.824369) (end 52.832 103.378) (stroke (width 0.05) (type solid)) (layer "Edge.Cuts"))
 (gr_line (start 52.832 147.32) (end 90.932 147.32) (stroke (width 0.05) (type solid)) (layer "Edge.Cuts"))
 (segment (start 100.887979 111.887979) (end 100.679378 111.887979) (width 0.25) (layer "F.Cu") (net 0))
 (segment (start 81.320622 131.679378) (end 81.429378 131.679378) (width 0.25) (layer "F.Cu") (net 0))
 (segment (start 81.320622 112.320622) (end 81.320622 112.179378) (width 0.25) (layer "F.Cu") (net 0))
 (segment (start 87 111) (end 91 111) (width 0.25) (layer "F.Cu") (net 3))
 (segment (start 83.9 107.9) (end 87 111) (width 0.25) (layer "F.Cu") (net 3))
 (segment (start 82.382486 107.9) (end 83.9 107.9) (width 0.25) (layer "F.Cu") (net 3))
 (segment (start 79.641243 110.641243) (end 82.382486 107.9) (width 0.25) (layer "F.Cu") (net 3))
 (segment (start 76.8 129.15) (end 79.9 126.05) (width 0.25) (layer "F.Cu") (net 5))
 (segment (start 79.541243 133.408757) (end 76.8 130.667514) (width 0.25) (layer "F.Cu") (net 5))
 (segment (start 79.9 126.05) (end 79.9 122.05) (width 0.25) (layer "F.Cu") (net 5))
 (segment (start 76.8 130.667514) (end 76.8 129.15) (width 0.25) (layer "F.Cu") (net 5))
 (segment (start 117.08 112.68) (end 117.08 110.14) (width 0.381) (layer "F.Cu") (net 7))
 (segment (start 117.08 135.54) (end 117.08 138.08) (width 0.381) (layer "F.Cu") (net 4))
 (segment (start 141.45 138.08) (end 141.45 135.54) (width 0.381) (layer "F.Cu") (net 1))
 (segment (start 141.48 110.11) (end 141.45 110.14) (width 0.25) (layer "F.Cu") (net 18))
 (segment (start 141.45 110.14) (end 141.45 112.68) (width 0.381) (layer "F.Cu") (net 18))
 (segment (start 105.3 113.082486) (end 105.3 114.6) (width 0.25) (layer "F.Cu") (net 6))
 (segment (start 102.2 117.7) (end 102.2 121.7) (width 0.25) (layer "F.Cu") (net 6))
 (segment (start 102.558757 110.341243) (end 105.3 113.082486) (width 0.25) (layer "F.Cu") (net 6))
 (segment (start 105.3 114.6) (end 102.2 117.7) (width 0.25) (layer "F.Cu") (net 6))
 (segment (start 102.258757 133.508757) (end 99.517514 136.25) (width 0.25) (layer "F.Cu") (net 2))
 (segment (start 99.517514 136.25) (end 98 136.25) (width 0.25) (layer "F.Cu") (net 2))
 (segment (start 94.9 133.15) (end 90.9 133.15) (width 0.25) (layer "F.Cu") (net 2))
 (segment (start 98 136.25) (end 94.9 133.15) (width 0.25) (layer "F.Cu") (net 2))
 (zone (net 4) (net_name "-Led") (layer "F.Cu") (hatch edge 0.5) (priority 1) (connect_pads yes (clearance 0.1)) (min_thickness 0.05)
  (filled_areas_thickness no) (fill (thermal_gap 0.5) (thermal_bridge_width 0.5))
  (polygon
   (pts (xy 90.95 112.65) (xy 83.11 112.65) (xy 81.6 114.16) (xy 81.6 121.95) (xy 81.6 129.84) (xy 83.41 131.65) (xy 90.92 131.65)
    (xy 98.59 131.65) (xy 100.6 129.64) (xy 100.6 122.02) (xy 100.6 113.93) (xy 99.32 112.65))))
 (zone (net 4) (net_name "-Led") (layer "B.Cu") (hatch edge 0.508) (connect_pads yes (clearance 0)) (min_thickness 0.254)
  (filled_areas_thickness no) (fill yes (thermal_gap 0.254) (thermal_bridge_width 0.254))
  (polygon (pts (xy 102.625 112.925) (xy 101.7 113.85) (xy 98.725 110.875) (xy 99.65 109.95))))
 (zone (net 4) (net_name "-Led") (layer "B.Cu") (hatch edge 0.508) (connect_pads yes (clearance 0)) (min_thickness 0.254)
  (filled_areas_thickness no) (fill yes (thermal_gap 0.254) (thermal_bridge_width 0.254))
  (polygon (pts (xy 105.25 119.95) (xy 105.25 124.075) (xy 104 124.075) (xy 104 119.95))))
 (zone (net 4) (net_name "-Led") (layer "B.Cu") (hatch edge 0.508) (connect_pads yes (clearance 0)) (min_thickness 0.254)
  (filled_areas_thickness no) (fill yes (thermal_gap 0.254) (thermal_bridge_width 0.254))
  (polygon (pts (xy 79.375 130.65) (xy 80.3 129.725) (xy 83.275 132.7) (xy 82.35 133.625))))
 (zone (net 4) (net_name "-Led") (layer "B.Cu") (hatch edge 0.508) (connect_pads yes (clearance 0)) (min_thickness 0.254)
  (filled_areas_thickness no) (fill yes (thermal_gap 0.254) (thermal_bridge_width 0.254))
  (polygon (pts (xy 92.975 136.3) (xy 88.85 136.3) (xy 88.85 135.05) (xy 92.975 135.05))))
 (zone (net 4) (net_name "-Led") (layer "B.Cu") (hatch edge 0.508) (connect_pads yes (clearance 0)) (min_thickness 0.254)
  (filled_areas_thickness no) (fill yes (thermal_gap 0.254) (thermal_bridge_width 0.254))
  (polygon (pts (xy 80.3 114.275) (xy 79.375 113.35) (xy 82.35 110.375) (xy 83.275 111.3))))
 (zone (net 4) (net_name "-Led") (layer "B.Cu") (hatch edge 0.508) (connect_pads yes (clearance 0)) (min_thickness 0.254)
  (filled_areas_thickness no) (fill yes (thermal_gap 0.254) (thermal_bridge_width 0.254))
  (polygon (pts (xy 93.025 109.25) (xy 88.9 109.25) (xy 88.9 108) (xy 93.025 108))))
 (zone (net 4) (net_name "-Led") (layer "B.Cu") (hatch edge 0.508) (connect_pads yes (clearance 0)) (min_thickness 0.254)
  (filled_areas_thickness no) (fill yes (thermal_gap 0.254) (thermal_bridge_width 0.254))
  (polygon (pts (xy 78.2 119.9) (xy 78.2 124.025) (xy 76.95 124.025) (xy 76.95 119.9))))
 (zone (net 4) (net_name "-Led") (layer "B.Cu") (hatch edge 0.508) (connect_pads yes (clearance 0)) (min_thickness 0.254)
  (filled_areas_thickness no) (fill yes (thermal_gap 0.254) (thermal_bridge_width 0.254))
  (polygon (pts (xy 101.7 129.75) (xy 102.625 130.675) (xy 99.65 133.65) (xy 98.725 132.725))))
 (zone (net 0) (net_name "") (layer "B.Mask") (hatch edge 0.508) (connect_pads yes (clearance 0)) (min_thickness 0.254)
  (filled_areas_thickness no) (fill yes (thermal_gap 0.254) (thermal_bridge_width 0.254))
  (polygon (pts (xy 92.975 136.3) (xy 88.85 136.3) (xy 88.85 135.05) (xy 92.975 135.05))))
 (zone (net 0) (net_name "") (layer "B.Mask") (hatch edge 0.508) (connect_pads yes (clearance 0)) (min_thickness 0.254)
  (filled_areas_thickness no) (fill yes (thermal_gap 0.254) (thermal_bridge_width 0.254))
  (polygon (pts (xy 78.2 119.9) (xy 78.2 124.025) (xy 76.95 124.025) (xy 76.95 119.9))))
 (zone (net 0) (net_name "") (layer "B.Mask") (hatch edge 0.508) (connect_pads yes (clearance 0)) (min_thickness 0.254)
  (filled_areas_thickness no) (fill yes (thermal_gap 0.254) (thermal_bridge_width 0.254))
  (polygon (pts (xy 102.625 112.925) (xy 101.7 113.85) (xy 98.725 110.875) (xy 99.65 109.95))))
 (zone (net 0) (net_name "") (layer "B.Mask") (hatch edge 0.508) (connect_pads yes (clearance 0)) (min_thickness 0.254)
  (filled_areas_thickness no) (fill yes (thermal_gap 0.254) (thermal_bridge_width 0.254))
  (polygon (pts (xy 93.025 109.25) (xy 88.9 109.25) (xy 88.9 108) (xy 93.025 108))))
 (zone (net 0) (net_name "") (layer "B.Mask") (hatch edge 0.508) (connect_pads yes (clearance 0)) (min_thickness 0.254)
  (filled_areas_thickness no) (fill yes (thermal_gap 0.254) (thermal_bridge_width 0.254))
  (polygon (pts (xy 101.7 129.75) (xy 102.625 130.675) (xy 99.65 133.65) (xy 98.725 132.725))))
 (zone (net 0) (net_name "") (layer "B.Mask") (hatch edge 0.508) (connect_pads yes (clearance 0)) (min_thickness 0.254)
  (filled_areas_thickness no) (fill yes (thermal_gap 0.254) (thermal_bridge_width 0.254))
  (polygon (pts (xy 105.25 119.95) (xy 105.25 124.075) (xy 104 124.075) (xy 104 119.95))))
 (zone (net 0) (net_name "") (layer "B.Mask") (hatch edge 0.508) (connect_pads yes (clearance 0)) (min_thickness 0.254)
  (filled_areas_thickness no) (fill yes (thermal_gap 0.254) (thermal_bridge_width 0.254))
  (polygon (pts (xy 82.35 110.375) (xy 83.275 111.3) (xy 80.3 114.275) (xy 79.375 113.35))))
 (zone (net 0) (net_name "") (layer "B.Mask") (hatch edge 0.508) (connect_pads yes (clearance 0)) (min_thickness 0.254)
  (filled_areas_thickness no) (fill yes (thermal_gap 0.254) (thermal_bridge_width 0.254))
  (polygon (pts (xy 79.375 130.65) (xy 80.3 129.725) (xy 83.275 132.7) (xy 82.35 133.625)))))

